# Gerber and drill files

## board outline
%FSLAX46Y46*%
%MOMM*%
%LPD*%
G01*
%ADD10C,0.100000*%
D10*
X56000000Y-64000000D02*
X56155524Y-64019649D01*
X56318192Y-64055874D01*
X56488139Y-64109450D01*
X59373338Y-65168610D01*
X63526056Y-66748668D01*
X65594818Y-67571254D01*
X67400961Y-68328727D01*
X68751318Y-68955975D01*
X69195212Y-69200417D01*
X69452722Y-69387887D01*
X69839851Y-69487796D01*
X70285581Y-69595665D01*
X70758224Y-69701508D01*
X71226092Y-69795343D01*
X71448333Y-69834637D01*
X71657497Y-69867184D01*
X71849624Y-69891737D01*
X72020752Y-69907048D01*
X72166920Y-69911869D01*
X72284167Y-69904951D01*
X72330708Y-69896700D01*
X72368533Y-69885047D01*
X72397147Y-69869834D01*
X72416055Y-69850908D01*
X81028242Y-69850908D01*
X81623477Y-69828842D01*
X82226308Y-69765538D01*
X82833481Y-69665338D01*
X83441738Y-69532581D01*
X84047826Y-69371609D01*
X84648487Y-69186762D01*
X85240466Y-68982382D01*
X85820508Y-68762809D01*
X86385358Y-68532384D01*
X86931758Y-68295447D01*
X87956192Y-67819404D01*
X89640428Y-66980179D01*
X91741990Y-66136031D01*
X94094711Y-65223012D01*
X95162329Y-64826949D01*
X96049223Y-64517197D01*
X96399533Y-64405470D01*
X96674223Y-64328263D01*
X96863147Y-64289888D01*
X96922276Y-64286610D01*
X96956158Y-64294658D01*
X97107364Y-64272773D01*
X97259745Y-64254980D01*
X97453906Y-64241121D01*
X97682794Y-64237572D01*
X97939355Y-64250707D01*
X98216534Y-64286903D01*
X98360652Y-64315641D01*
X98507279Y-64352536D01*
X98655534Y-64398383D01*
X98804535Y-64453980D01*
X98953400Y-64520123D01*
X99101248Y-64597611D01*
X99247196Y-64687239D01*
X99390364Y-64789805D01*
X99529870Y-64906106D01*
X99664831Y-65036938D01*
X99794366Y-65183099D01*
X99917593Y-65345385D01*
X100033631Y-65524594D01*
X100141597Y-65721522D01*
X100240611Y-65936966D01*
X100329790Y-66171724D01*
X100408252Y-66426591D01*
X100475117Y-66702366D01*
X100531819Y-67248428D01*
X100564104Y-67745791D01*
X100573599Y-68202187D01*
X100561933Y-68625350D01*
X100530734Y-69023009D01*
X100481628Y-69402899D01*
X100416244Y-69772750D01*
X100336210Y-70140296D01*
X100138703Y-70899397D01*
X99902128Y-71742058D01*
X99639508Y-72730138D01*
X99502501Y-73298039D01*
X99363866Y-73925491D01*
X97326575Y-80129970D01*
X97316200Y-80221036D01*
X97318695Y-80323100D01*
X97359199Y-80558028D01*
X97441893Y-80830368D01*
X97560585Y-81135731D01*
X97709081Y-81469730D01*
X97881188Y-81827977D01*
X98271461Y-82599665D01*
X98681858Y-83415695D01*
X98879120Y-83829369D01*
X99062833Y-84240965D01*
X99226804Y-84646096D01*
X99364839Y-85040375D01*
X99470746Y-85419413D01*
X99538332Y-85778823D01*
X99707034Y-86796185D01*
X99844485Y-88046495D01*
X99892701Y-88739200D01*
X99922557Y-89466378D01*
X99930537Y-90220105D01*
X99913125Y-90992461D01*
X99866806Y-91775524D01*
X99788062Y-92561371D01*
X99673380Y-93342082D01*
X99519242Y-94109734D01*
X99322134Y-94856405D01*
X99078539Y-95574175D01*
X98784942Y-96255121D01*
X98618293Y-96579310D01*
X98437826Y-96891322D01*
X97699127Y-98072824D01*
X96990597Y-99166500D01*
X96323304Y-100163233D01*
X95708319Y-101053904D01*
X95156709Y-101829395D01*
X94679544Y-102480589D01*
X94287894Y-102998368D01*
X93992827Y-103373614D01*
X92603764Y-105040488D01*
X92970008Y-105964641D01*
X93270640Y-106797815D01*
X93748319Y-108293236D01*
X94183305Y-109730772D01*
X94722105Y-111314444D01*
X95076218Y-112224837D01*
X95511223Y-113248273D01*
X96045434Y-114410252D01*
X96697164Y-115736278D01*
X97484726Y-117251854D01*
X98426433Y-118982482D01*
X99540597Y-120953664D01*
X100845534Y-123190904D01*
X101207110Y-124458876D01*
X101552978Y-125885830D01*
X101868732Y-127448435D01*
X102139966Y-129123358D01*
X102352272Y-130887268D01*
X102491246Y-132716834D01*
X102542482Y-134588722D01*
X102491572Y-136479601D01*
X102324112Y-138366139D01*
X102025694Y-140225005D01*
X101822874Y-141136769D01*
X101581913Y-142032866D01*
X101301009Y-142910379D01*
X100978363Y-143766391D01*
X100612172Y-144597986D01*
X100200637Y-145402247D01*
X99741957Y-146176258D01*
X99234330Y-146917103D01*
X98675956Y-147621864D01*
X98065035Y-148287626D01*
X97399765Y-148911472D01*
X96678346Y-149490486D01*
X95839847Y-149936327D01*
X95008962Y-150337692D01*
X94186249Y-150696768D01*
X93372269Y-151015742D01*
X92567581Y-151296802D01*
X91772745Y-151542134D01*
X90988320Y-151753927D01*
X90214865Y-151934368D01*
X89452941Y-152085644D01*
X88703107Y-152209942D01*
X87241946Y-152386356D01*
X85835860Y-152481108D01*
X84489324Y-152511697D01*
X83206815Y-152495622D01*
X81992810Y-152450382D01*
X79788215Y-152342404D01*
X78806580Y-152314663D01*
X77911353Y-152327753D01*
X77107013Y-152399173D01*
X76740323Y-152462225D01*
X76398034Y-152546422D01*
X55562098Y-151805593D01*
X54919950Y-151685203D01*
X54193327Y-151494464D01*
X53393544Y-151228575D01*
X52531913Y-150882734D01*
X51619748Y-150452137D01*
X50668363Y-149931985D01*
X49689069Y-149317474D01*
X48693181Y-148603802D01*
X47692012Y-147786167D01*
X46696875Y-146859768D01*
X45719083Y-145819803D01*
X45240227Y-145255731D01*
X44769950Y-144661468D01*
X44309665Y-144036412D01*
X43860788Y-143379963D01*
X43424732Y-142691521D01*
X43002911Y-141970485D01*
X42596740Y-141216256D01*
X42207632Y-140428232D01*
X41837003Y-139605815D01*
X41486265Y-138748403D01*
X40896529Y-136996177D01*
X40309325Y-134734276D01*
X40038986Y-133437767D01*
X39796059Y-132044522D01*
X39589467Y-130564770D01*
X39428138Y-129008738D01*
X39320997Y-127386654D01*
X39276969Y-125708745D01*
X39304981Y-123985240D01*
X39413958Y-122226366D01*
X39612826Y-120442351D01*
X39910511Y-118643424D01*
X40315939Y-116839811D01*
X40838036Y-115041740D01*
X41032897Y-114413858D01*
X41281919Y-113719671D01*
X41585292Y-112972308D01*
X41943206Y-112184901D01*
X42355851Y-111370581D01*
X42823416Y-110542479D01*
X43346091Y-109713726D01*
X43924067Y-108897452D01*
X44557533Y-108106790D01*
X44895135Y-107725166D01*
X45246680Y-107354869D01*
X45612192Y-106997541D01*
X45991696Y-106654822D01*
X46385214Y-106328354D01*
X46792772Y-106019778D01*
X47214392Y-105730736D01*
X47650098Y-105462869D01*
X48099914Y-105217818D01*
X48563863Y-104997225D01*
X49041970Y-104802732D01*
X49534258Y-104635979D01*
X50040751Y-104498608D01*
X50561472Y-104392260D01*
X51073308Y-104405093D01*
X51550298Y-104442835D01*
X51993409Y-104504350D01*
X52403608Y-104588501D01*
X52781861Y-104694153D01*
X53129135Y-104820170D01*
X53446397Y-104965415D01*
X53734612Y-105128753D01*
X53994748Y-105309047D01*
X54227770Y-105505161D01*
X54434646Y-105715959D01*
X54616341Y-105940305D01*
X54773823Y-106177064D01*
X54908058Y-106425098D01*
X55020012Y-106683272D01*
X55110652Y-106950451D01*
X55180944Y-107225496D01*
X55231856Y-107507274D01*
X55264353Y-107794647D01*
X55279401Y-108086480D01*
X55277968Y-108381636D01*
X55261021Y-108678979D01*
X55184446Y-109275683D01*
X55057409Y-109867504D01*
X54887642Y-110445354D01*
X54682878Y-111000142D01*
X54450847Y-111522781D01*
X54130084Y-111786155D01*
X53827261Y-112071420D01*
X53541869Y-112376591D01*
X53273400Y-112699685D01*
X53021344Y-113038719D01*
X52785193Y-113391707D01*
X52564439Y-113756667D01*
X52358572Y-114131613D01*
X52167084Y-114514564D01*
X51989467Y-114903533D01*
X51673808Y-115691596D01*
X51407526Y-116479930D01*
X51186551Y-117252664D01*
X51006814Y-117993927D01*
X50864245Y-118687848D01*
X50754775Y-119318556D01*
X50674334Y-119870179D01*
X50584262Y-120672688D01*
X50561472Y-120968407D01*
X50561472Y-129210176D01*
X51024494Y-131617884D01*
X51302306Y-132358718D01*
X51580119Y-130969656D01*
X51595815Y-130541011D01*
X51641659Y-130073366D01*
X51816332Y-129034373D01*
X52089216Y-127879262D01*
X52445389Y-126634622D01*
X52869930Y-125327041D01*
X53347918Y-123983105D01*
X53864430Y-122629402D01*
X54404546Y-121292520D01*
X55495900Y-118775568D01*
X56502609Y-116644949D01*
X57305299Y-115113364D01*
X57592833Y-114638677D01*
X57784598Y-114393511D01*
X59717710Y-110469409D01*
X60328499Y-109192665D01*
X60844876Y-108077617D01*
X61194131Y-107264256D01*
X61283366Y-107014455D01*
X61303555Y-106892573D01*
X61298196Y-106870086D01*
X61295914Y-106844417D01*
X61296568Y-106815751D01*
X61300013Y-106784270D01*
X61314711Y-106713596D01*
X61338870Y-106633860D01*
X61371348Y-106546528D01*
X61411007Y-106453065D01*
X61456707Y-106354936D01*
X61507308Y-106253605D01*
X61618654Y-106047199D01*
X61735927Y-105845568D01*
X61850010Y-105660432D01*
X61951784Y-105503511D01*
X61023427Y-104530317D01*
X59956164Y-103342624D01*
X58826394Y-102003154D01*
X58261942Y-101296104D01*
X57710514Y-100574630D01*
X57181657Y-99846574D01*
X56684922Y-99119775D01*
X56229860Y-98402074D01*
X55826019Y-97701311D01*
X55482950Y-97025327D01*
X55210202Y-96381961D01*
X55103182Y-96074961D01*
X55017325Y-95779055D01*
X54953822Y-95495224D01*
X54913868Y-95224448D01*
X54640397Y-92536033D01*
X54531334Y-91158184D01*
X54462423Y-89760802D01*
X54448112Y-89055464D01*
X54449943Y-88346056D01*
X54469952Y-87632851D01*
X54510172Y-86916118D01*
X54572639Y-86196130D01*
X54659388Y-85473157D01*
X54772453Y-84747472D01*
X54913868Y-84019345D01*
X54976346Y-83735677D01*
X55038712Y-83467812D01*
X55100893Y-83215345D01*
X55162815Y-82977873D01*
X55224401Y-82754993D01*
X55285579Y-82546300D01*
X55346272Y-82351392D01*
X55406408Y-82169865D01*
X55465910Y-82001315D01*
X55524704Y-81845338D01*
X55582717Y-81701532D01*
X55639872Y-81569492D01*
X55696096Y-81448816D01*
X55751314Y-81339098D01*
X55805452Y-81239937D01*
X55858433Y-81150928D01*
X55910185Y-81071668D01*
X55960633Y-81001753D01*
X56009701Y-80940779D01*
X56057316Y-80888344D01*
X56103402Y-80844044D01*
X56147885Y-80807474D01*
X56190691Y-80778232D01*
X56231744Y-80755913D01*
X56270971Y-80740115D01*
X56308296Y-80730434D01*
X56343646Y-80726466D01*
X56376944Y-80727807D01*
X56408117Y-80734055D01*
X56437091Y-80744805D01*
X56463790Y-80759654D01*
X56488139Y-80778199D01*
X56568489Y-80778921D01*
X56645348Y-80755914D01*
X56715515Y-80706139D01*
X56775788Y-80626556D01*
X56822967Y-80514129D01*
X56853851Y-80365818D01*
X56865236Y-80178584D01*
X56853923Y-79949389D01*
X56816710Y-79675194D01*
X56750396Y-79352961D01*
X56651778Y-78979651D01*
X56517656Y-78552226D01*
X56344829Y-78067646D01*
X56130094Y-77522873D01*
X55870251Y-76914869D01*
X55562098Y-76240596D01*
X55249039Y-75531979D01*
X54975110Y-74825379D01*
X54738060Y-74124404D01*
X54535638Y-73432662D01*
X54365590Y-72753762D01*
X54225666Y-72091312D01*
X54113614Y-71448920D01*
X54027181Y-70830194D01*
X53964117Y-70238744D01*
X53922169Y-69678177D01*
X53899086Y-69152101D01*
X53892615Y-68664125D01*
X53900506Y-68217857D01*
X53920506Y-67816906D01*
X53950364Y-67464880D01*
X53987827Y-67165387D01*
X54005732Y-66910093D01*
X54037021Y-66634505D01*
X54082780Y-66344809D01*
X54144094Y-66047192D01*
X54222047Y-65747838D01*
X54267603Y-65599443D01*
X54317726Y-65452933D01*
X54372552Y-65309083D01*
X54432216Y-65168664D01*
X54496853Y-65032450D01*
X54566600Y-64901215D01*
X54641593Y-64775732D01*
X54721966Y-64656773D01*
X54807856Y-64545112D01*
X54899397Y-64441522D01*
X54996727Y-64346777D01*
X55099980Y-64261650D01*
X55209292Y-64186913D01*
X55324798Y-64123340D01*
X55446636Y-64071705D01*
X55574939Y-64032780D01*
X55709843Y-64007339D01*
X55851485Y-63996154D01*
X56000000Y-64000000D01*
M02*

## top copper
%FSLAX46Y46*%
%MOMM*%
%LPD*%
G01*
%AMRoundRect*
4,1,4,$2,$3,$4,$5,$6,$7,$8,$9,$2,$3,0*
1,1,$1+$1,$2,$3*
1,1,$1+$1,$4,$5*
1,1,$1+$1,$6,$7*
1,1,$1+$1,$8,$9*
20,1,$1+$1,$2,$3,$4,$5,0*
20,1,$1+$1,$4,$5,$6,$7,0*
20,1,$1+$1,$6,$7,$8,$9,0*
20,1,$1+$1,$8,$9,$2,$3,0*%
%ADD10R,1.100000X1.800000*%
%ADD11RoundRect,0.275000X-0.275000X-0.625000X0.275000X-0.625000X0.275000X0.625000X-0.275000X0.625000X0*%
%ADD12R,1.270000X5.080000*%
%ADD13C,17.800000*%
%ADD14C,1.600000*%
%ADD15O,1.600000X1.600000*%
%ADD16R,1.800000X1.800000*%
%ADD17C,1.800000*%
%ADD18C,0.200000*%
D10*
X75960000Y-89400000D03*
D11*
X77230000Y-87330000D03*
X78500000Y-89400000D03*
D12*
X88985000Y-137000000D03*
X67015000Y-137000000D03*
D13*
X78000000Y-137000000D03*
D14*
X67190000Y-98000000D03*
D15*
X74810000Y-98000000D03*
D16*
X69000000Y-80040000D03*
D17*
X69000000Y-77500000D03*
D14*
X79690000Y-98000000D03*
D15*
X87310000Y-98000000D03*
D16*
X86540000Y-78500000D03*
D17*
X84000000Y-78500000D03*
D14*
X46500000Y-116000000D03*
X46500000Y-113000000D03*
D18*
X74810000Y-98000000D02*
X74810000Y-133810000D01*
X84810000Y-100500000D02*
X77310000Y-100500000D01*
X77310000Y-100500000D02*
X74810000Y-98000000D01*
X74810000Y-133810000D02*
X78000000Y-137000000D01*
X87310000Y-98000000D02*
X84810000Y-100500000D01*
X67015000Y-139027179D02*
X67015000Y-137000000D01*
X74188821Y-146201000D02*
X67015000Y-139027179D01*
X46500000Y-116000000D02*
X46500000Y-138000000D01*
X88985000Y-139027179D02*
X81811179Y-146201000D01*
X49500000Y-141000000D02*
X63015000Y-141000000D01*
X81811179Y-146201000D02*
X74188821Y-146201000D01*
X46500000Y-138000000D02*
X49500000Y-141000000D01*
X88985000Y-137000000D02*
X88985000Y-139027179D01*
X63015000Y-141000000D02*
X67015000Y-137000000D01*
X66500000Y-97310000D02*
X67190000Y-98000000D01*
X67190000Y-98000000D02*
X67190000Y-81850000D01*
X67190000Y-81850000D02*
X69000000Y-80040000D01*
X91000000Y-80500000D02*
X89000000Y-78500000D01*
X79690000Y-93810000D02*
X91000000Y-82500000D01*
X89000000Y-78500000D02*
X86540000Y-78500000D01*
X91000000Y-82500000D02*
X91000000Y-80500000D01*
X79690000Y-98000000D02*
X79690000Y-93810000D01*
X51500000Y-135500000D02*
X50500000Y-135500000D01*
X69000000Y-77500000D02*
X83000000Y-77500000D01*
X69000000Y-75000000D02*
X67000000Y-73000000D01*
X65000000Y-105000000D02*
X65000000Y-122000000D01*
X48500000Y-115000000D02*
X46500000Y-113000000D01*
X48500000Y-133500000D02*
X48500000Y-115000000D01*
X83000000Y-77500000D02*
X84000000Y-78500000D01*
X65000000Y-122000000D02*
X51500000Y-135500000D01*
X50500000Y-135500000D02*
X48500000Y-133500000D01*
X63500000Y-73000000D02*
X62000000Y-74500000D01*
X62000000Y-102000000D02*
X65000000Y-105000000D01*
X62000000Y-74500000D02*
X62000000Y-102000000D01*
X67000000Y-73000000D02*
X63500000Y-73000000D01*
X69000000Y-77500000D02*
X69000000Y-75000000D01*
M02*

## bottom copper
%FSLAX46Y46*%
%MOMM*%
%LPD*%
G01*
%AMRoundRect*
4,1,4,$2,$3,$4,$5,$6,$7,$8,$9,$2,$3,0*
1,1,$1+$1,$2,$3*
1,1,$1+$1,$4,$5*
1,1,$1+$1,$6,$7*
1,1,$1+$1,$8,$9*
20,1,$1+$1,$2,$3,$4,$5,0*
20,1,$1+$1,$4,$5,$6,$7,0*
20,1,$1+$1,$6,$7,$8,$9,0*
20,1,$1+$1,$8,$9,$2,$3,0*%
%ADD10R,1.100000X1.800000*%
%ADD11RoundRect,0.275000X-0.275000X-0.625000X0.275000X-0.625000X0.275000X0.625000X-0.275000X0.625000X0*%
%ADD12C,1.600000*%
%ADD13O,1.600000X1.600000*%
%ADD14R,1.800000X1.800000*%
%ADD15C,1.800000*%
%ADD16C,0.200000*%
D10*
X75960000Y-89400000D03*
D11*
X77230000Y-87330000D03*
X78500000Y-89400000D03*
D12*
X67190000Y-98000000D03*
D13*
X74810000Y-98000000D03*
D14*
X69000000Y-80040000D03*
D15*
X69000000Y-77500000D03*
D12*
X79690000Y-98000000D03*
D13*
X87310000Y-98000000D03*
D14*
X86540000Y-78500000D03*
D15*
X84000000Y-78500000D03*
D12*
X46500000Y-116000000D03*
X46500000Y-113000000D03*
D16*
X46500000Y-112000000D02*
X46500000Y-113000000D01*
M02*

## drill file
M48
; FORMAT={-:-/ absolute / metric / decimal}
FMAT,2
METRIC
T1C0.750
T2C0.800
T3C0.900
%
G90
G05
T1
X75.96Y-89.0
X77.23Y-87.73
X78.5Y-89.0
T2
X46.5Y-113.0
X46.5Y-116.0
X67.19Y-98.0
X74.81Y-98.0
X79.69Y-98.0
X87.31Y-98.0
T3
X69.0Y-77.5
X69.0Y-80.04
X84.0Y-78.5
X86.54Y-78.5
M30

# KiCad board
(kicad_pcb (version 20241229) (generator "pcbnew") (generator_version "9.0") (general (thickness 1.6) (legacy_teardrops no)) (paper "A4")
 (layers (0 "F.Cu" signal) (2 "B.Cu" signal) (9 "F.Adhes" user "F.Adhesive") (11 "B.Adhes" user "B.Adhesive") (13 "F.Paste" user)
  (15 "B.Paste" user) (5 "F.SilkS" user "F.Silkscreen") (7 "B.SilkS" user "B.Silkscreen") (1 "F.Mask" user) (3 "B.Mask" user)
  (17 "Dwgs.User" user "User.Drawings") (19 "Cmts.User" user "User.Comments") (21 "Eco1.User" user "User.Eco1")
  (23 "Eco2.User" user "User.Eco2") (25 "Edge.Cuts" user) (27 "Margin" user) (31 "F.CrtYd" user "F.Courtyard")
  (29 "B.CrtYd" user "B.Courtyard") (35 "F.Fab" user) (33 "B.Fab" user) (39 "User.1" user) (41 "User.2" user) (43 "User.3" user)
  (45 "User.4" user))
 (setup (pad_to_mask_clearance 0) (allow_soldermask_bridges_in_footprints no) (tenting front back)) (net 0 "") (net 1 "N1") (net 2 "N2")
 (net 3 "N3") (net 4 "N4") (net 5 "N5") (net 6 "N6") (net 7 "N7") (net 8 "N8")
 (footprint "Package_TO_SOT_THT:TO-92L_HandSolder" (layer "F.Cu") (at 75.96 89)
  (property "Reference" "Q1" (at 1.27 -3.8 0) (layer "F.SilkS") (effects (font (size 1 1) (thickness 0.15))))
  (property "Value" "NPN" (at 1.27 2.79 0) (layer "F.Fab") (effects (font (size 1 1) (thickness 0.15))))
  (pad "1" thru_hole rect (at 0 0) (size 1.1 1.8) (drill 0.75 (offset 0 0.4)) (layers "*.Cu" "*.Mask") (remove_unused_layers no)
   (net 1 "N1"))
  (pad "2" thru_hole roundrect (at 1.27 -1.27) (size 1.1 1.8) (drill 0.75 (offset 0 -0.4)) (layers "*.Cu" "*.Mask")
   (remove_unused_layers no) (roundrect_rratio 0.25) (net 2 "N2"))
  (pad "3" thru_hole roundrect (at 2.54 0) (size 1.1 1.8) (drill 0.75 (offset 0 0.4)) (layers "*.Cu" "*.Mask") (remove_unused_layers no)
   (roundrect_rratio 0.25) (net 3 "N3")))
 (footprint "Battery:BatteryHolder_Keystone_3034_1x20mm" (layer "F.Cu") (at 78 137 180)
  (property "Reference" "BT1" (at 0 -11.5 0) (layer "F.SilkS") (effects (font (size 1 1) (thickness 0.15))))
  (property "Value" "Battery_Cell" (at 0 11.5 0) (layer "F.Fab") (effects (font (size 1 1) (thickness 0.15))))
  (pad "1" smd rect (at -10.985 0 180) (size 1.27 5.08) (layers "F.Cu" "F.Mask" "F.Paste") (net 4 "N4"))
  (pad "1" smd rect (at 10.985 0 180) (size 1.27 5.08) (layers "F.Cu" "F.Mask" "F.Paste") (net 4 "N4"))
  (pad "2" smd circle (at 0 0 180) (size 17.8 17.8) (layers "F.Cu" "F.Mask") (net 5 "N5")))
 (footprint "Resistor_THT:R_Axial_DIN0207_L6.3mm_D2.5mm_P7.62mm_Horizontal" (layer "F.Cu") (at 67.19 98)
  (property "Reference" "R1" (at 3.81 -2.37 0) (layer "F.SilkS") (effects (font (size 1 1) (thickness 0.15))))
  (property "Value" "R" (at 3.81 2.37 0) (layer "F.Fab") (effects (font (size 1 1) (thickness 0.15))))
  (pad "1" thru_hole circle (at 0 0) (size 1.6 1.6) (drill 0.8) (layers "*.Cu" "*.Mask") (remove_unused_layers no) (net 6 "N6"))
  (pad "2" thru_hole oval (at 7.62 0) (size 1.6 1.6) (drill 0.8) (layers "*.Cu" "*.Mask") (remove_unused_layers no) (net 5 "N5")))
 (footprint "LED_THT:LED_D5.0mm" (layer "F.Cu") (at 69 80.04 90)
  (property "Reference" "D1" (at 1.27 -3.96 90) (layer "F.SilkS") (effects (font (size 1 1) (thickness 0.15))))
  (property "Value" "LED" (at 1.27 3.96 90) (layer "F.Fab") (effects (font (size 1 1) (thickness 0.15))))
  (pad "1" thru_hole rect (at 0 0 90) (size 1.8 1.8) (drill 0.9) (layers "*.Cu" "*.Mask") (remove_unused_layers no) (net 6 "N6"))
  (pad "2" thru_hole circle (at 2.54 0 90) (size 1.8 1.8) (drill 0.9) (layers "*.Cu" "*.Mask") (remove_unused_layers no) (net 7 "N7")))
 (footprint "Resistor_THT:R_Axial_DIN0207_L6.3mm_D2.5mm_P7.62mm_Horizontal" (layer "F.Cu") (at 79.69 98)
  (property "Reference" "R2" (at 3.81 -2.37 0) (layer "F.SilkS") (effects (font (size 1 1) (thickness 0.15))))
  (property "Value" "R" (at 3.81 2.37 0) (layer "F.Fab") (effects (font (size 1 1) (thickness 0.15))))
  (pad "1" thru_hole circle (at 0 0) (size 1.6 1.6) (drill 0.8) (layers "*.Cu" "*.Mask") (remove_unused_layers no) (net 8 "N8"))
  (pad "2" thru_hole oval (at 7.62 0) (size 1.6 1.6) (drill 0.8) (layers "*.Cu" "*.Mask") (remove_unused_layers no) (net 5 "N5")))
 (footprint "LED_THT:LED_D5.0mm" (layer "F.Cu") (at 86.54 78.5 180)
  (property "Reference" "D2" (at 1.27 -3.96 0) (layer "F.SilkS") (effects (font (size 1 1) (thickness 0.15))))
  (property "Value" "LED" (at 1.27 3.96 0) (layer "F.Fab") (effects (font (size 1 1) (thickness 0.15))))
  (pad "1" thru_hole rect (at 0 0 180) (size 1.8 1.8) (drill 0.9) (layers "*.Cu" "*.Mask") (remove_unused_layers no) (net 8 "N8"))
  (pad "2" thru_hole circle (at 2.54 0 180) (size 1.8 1.8) (drill 0.9) (layers "*.Cu" "*.Mask") (remove_unused_layers no) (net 7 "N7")))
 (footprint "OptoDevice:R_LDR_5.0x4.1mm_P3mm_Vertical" (layer "F.Cu") (at 46.5 116 90)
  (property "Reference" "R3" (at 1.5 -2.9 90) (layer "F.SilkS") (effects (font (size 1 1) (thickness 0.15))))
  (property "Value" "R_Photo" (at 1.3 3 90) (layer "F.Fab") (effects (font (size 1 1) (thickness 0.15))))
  (pad "1" thru_hole circle (at 0 0 90) (size 1.6 1.6) (drill 0.8) (layers "*.Cu" "*.Mask") (remove_unused_layers no) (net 4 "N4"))
  (pad "2" thru_hole circle (at 3 0 90) (size 1.6 1.6) (drill 0.8) (layers "*.Cu" "*.Mask") (remove_unused_layers no) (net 7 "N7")))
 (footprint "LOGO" (layer "B.Cu") (at 83.5 77.5 180)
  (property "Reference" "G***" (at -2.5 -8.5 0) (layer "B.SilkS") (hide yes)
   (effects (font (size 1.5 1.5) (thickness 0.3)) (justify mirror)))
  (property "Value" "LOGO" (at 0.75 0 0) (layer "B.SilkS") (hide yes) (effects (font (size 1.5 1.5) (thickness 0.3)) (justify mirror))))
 (gr_poly
  (pts (xy 56 64) (xy 56.155524 64.019649) (xy 56.318192 64.055874) (xy 56.488139 64.10945) (xy 59.373338 65.16861) (xy 63.526056 66.748668)
   (xy 65.594818 67.571254) (xy 67.400961 68.328727) (xy 68.751318 68.955975) (xy 69.195212 69.200417) (xy 69.452722 69.387887)
   (xy 69.839851 69.487796) (xy 70.285581 69.595665) (xy 70.758224 69.701508) (xy 71.226092 69.795343) (xy 71.448333 69.834637)
   (xy 71.657497 69.867184) (xy 71.849624 69.891737) (xy 72.020752 69.907048) (xy 72.16692 69.911869) (xy 72.284167 69.904951)
   (xy 72.330708 69.8967) (xy 72.368533 69.885047) (xy 72.397147 69.869834) (xy 72.416055 69.850908) (xy 81.028242 69.850908)
   (xy 81.623477 69.828842) (xy 82.226308 69.765538) (xy 82.833481 69.665338) (xy 83.441738 69.532581) (xy 84.047826 69.371609)
   (xy 84.648487 69.186762) (xy 85.240466 68.982382) (xy 85.820508 68.762809) (xy 86.385358 68.532384) (xy 86.931758 68.295447)
   (xy 87.956192 67.819404) (xy 89.640428 66.980179) (xy 91.74199 66.136031) (xy 94.094711 65.223012) (xy 95.162329 64.826949)
   (xy 96.049223 64.517197) (xy 96.399533 64.40547) (xy 96.674223 64.328263) (xy 96.863147 64.289888) (xy 96.922276 64.28661)
   (xy 96.956158 64.294658) (xy 97.107364 64.272773) (xy 97.259745 64.25498) (xy 97.453906 64.241121) (xy 97.682794 64.237572)
   (xy 97.939355 64.250707) (xy 98.216534 64.286903) (xy 98.360652 64.315641) (xy 98.507279 64.352536) (xy 98.655534 64.398383)
   (xy 98.804535 64.45398) (xy 98.9534 64.520123) (xy 99.101248 64.597611) (xy 99.247196 64.687239) (xy 99.390364 64.789805)
   (xy 99.52987 64.906106) (xy 99.664831 65.036938) (xy 99.794366 65.183099) (xy 99.917593 65.345385) (xy 100.033631 65.524594)
   (xy 100.141597 65.721522) (xy 100.240611 65.936966) (xy 100.32979 66.171724) (xy 100.408252 66.426591) (xy 100.475117 66.702366)
   (xy 100.531819 67.248428) (xy 100.564104 67.745791) (xy 100.573599 68.202187) (xy 100.561933 68.62535) (xy 100.530734 69.023009)
   (xy 100.481628 69.402899) (xy 100.416244 69.77275) (xy 100.33621 70.140296) (xy 100.138703 70.899397) (xy 99.902128 71.742058)
   (xy 99.639508 72.730138) (xy 99.502501 73.298039) (xy 99.363866 73.925491) (xy 97.326575 80.12997) (xy 97.3162 80.221036)
   (xy 97.318695 80.3231) (xy 97.359199 80.558028) (xy 97.441893 80.830368) (xy 97.560585 81.135731) (xy 97.709081 81.46973)
   (xy 97.881188 81.827977) (xy 98.271461 82.599665) (xy 98.681858 83.415695) (xy 98.87912 83.829369) (xy 99.062833 84.240965)
   (xy 99.226804 84.646096) (xy 99.364839 85.040375) (xy 99.470746 85.419413) (xy 99.538332 85.778823) (xy 99.707034 86.796185)
   (xy 99.844485 88.046495) (xy 99.892701 88.7392) (xy 99.922557 89.466378) (xy 99.930537 90.220105) (xy 99.913125 90.992461)
   (xy 99.866806 91.775524) (xy 99.788062 92.561371) (xy 99.67338 93.342082) (xy 99.519242 94.109734) (xy 99.322134 94.856405)
   (xy 99.078539 95.574175) (xy 98.784942 96.255121) (xy 98.618293 96.57931) (xy 98.437826 96.891322) (xy 97.699127 98.072824)
   (xy 96.990597 99.1665) (xy 96.323304 100.163233) (xy 95.708319 101.053904) (xy 95.156709 101.829395) (xy 94.679544 102.480589)
   (xy 94.287894 102.998368) (xy 93.992827 103.373614) (xy 92.603764 105.040488) (xy 92.970008 105.964641) (xy 93.27064 106.797815)
   (xy 93.748319 108.293236) (xy 94.183305 109.730772) (xy 94.722105 111.314444) (xy 95.076218 112.224837) (xy 95.511223 113.248273)
   (xy 96.045434 114.410252) (xy 96.697164 115.736278) (xy 97.484726 117.251854) (xy 98.426433 118.982482) (xy 99.540597 120.953664)
   (xy 100.845534 123.190904) (xy 101.20711 124.458876) (xy 101.552978 125.88583) (xy 101.868732 127.448435) (xy 102.139966 129.123358)
   (xy 102.352272 130.887268) (xy 102.491246 132.716834) (xy 102.542482 134.588722) (xy 102.491572 136.479601) (xy 102.324112 138.366139)
   (xy 102.025694 140.225005) (xy 101.822874 141.136769) (xy 101.581913 142.032866) (xy 101.301009 142.910379) (xy 100.978363 143.766391)
   (xy 100.612172 144.597986) (xy 100.200637 145.402247) (xy 99.741957 146.176258) (xy 99.23433 146.917103) (xy 98.675956 147.621864)
   (xy 98.065035 148.287626) (xy 97.399765 148.911472) (xy 96.678346 149.490486) (xy 95.839847 149.936327) (xy 95.008962 150.337692)
   (xy 94.186249 150.696768) (xy 93.372269 151.015742) (xy 92.567581 151.296802) (xy 91.772745 151.542134) (xy 90.98832 151.753927)
   (xy 90.214865 151.934368) (xy 89.452941 152.085644) (xy 88.703107 152.209942) (xy 87.241946 152.386356) (xy 85.83586 152.481108)
   (xy 84.489324 152.511697) (xy 83.206815 152.495622) (xy 81.99281 152.450382) (xy 79.788215 152.342404) (xy 78.80658 152.314663)
   (xy 77.911353 152.327753) (xy 77.107013 152.399173) (xy 76.740323 152.462225) (xy 76.398034 152.546422) (xy 55.562098 151.805593)
   (xy 54.91995 151.685203) (xy 54.193327 151.494464) (xy 53.393544 151.228575) (xy 52.531913 150.882734) (xy 51.619748 150.452137)
   (xy 50.668363 149.931985) (xy 49.689069 149.317474) (xy 48.693181 148.603802) (xy 47.692012 147.786167) (xy 46.696875 146.859768)
   (xy 45.719083 145.819803) (xy 45.240227 145.255731) (xy 44.76995 144.661468) (xy 44.309665 144.036412) (xy 43.860788 143.379963)
   (xy 43.424732 142.691521) (xy 43.002911 141.970485) (xy 42.59674 141.216256) (xy 42.207632 140.428232) (xy 41.837003 139.605815)
   (xy 41.486265 138.748403) (xy 40.896529 136.996177) (xy 40.309325 134.734276) (xy 40.038986 133.437767) (xy 39.796059 132.044522)
   (xy 39.589467 130.56477) (xy 39.428138 129.008738) (xy 39.320997 127.386654) (xy 39.276969 125.708745) (xy 39.304981 123.98524)
   (xy 39.413958 122.226366) (xy 39.612826 120.442351) (xy 39.910511 118.643424) (xy 40.315939 116.839811) (xy 40.838036 115.04174)
   (xy 41.032897 114.413858) (xy 41.281919 113.719671) (xy 41.585292 112.972308) (xy 41.943206 112.184901) (xy 42.355851 111.370581)
   (xy 42.823416 110.542479) (xy 43.346091 109.713726) (xy 43.924067 108.897452) (xy 44.557533 108.10679) (xy 44.895135 107.725166)
   (xy 45.24668 107.354869) (xy 45.612192 106.997541) (xy 45.991696 106.654822) (xy 46.385214 106.328354) (xy 46.792772 106.019778)
   (xy 47.214392 105.730736) (xy 47.650098 105.462869) (xy 48.099914 105.217818) (xy 48.563863 104.997225) (xy 49.04197 104.802732)
   (xy 49.534258 104.635979) (xy 50.040751 104.498608) (xy 50.561472 104.39226) (xy 51.073308 104.405093) (xy 51.550298 104.442835)
   (xy 51.993409 104.50435) (xy 52.403608 104.588501) (xy 52.781861 104.694153) (xy 53.129135 104.82017) (xy 53.446397 104.965415)
   (xy 53.734612 105.128753) (xy 53.994748 105.309047) (xy 54.22777 105.505161) (xy 54.434646 105.715959) (xy 54.616341 105.940305)
   (xy 54.773823 106.177064) (xy 54.908058 106.425098) (xy 55.020012 106.683272) (xy 55.110652 106.950451) (xy 55.180944 107.225496)
   (xy 55.231856 107.507274) (xy 55.264353 107.794647) (xy 55.279401 108.08648) (xy 55.277968 108.381636) (xy 55.261021 108.678979)
   (xy 55.184446 109.275683) (xy 55.057409 109.867504) (xy 54.887642 110.445354) (xy 54.682878 111.000142) (xy 54.450847 111.522781)
   (xy 54.130084 111.786155) (xy 53.827261 112.07142) (xy 53.541869 112.376591) (xy 53.2734 112.699685) (xy 53.021344 113.038719)
   (xy 52.785193 113.391707) (xy 52.564439 113.756667) (xy 52.358572 114.131613) (xy 52.167084 114.514564) (xy 51.989467 114.903533)
   (xy 51.673808 115.691596) (xy 51.407526 116.47993) (xy 51.186551 117.252664) (xy 51.006814 117.993927) (xy 50.864245 118.687848)
   (xy 50.754775 119.318556) (xy 50.674334 119.870179) (xy 50.584262 120.672688) (xy 50.561472 120.968407) (xy 50.561472 129.210176)
   (xy 51.024494 131.617884) (xy 51.302306 132.358718) (xy 51.580119 130.969656) (xy 51.595815 130.541011) (xy 51.641659 130.073366)
   (xy 51.816332 129.034373) (xy 52.089216 127.879262) (xy 52.445389 126.634622) (xy 52.86993 125.327041) (xy 53.347918 123.983105)
   (xy 53.86443 122.629402) (xy 54.404546 121.29252) (xy 55.4959 118.775568) (xy 56.502609 116.644949) (xy 57.305299 115.113364)
   (xy 57.592833 114.638677) (xy 57.784598 114.393511) (xy 59.71771 110.469409) (xy 60.328499 109.192665) (xy 60.844876 108.077617)
   (xy 61.194131 107.264256) (xy 61.283366 107.014455) (xy 61.303555 106.892573) (xy 61.298196 106.870086) (xy 61.295914 106.844417)
   (xy 61.296568 106.815751) (xy 61.300013 106.78427) (xy 61.314711 106.713596) (xy 61.33887 106.63386) (xy 61.371348 106.546528)
   (xy 61.411007 106.453065) (xy 61.456707 106.354936) (xy 61.507308 106.253605) (xy 61.618654 106.047199) (xy 61.735927 105.845568)
   (xy 61.85001 105.660432) (xy 61.951784 105.503511) (xy 61.023427 104.530317) (xy 59.956164 103.342624) (xy 58.826394 102.003154)
   (xy 58.261942 101.296104) (xy 57.710514 100.57463) (xy 57.181657 99.846574) (xy 56.684922 99.119775) (xy 56.22986 98.402074)
   (xy 55.826019 97.701311) (xy 55.48295 97.025327) (xy 55.210202 96.381961) (xy 55.103182 96.074961) (xy 55.017325 95.779055)
   (xy 54.953822 95.495224) (xy 54.913868 95.224448) (xy 54.640397 92.536033) (xy 54.531334 91.158184) (xy 54.462423 89.760802)
   (xy 54.448112 89.055464) (xy 54.449943 88.346056) (xy 54.469952 87.632851) (xy 54.510172 86.916118) (xy 54.572639 86.19613)
   (xy 54.659388 85.473157) (xy 54.772453 84.747472) (xy 54.913868 84.019345) (xy 54.976346 83.735677) (xy 55.038712 83.467812)
   (xy 55.100893 83.215345) (xy 55.162815 82.977873) (xy 55.224401 82.754993) (xy 55.285579 82.5463) (xy 55.346272 82.351392)
   (xy 55.406408 82.169865) (xy 55.46591 82.001315) (xy 55.524704 81.845338) (xy 55.582717 81.701532) (xy 55.639872 81.569492)
   (xy 55.696096 81.448816) (xy 55.751314 81.339098) (xy 55.805452 81.239937) (xy 55.858433 81.150928) (xy 55.910185 81.071668)
   (xy 55.960633 81.001753) (xy 56.009701 80.940779) (xy 56.057316 80.888344) (xy 56.103402 80.844044) (xy 56.147885 80.807474)
   (xy 56.190691 80.778232) (xy 56.231744 80.755913) (xy 56.270971 80.740115) (xy 56.308296 80.730434) (xy 56.343646 80.726466)
   (xy 56.376944 80.727807) (xy 56.408117 80.734055) (xy 56.437091 80.744805) (xy 56.46379 80.759654) (xy 56.488139 80.778199)
   (xy 56.568489 80.778921) (xy 56.645348 80.755914) (xy 56.715515 80.706139) (xy 56.775788 80.626556) (xy 56.822967 80.514129)
   (xy 56.853851 80.365818) (xy 56.865236 80.178584) (xy 56.853923 79.949389) (xy 56.81671 79.675194) (xy 56.750396 79.352961)
   (xy 56.651778 78.979651) (xy 56.517656 78.552226) (xy 56.344829 78.067646) (xy 56.130094 77.522873) (xy 55.870251 76.914869)
   (xy 55.562098 76.240596) (xy 55.249039 75.531979) (xy 54.97511 74.825379) (xy 54.73806 74.124404) (xy 54.535638 73.432662)
   (xy 54.36559 72.753762) (xy 54.225666 72.091312) (xy 54.113614 71.44892) (xy 54.027181 70.830194) (xy 53.964117 70.238744)
   (xy 53.922169 69.678177) (xy 53.899086 69.152101) (xy 53.892615 68.664125) (xy 53.900506 68.217857) (xy 53.920506 67.816906)
   (xy 53.950364 67.46488) (xy 53.987827 67.165387) (xy 54.005732 66.910093) (xy 54.037021 66.634505) (xy 54.08278 66.344809)
   (xy 54.144094 66.047192) (xy 54.222047 65.747838) (xy 54.267603 65.599443) (xy 54.317726 65.452933) (xy 54.372552 65.309083)
   (xy 54.432216 65.168664) (xy 54.496853 65.03245) (xy 54.5666 64.901215) (xy 54.641593 64.775732) (xy 54.721966 64.656773)
   (xy 54.807856 64.545112) (xy 54.899397 64.441522) (xy 54.996727 64.346777) (xy 55.09998 64.26165) (xy 55.209292 64.186913)
   (xy 55.324798 64.12334) (xy 55.446636 64.071705) (xy 55.574939 64.03278) (xy 55.709843 64.007339) (xy 55.851485 63.996154))
  (stroke (width 0.1) (type solid) (color 255 0 0 1)) (fill no) (layer "Edge.Cuts"))
 (segment (start 74.81 98) (end 74.81 133.81) (width 0.2) (layer "F.Cu") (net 5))
 (segment (start 84.81 100.5) (end 77.31 100.5) (width 0.2) (layer "F.Cu") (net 5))
 (segment (start 77.31 100.5) (end 74.81 98) (width 0.2) (layer "F.Cu") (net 5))
 (segment (start 74.81 133.81) (end 78 137) (width 0.2) (layer "F.Cu") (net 5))
 (segment (start 87.31 98) (end 84.81 100.5) (width 0.2) (layer "F.Cu") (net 5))
 (segment (start 67.015 139.027179) (end 67.015 137) (width 0.2) (layer "F.Cu") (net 4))
 (segment (start 74.188821 146.201) (end 67.015 139.027179) (width 0.2) (layer "F.Cu") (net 4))
 (segment (start 46.5 116) (end 46.5 138) (width 0.2) (layer "F.Cu") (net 4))
 (segment (start 88.985 139.027179) (end 81.811179 146.201) (width 0.2) (layer "F.Cu") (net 4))
 (segment (start 49.5 141) (end 63.015 141) (width 0.2) (layer "F.Cu") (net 4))
 (segment (start 81.811179 146.201) (end 74.188821 146.201) (width 0.2) (layer "F.Cu") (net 4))
 (segment (start 46.5 138) (end 49.5 141) (width 0.2) (layer "F.Cu") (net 4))
 (segment (start 88.985 137) (end 88.985 139.027179) (width 0.2) (layer "F.Cu") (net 4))
 (segment (start 63.015 141) (end 67.015 137) (width 0.2) (layer "F.Cu") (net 4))
 (segment (start 66.5 97.31) (end 67.19 98) (width 0.2) (layer "F.Cu") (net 6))
 (segment (start 67.19 98) (end 67.19 81.85) (width 0.2) (layer "F.Cu") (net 6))
 (segment (start 67.19 81.85) (end 69 80.04) (width 0.2) (layer "F.Cu") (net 6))
 (segment (start 91 80.5) (end 89 78.5) (width 0.2) (layer "F.Cu") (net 8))
 (segment (start 79.69 93.81) (end 91 82.5) (width 0.2) (layer "F.Cu") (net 8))
 (segment (start 89 78.5) (end 86.54 78.5) (width 0.2) (layer "F.Cu") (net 8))
 (segment (start 91 82.5) (end 91 80.5) (width 0.2) (layer "F.Cu") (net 8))
 (segment (start 79.69 98) (end 79.69 93.81) (width 0.2) (layer "F.Cu") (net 8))
 (segment (start 51.5 135.5) (end 50.5 135.5) (width 0.2) (layer "F.Cu") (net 7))
 (segment (start 69 77.5) (end 83 77.5) (width 0.2) (layer "F.Cu") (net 7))
 (segment (start 69 75) (end 67 73) (width 0.2) (layer "F.Cu") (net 7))
 (segment (start 65 105) (end 65 122) (width 0.2) (layer "F.Cu") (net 7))
 (segment (start 48.5 115) (end 46.5 113) (width 0.2) (layer "F.Cu") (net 7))
 (segment (start 48.5 133.5) (end 48.5 115) (width 0.2) (layer "F.Cu") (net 7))
 (segment (start 83 77.5) (end 84 78.5) (width 0.2) (layer "F.Cu") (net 7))
 (segment (start 65 122) (end 51.5 135.5) (width 0.2) (layer "F.Cu") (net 7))
 (segment (start 50.5 135.5) (end 48.5 133.5) (width 0.2) (layer "F.Cu") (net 7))
 (segment (start 63.5 73) (end 62 74.5) (width 0.2) (layer "F.Cu") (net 7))
 (segment (start 62 102) (end 65 105) (width 0.2) (layer "F.Cu") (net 7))
 (segment (start 62 74.5) (end 62 102) (width 0.2) (layer "F.Cu") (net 7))
 (segment (start 67 73) (end 63.5 73) (width 0.2) (layer "F.Cu") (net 7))
 (segment (start 69 77.5) (end 69 75) (width 0.2) (layer "F.Cu") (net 7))
 (segment (start 46.5 112) (end 46.5 113) (width 0.2) (layer "B.Cu") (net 7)))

